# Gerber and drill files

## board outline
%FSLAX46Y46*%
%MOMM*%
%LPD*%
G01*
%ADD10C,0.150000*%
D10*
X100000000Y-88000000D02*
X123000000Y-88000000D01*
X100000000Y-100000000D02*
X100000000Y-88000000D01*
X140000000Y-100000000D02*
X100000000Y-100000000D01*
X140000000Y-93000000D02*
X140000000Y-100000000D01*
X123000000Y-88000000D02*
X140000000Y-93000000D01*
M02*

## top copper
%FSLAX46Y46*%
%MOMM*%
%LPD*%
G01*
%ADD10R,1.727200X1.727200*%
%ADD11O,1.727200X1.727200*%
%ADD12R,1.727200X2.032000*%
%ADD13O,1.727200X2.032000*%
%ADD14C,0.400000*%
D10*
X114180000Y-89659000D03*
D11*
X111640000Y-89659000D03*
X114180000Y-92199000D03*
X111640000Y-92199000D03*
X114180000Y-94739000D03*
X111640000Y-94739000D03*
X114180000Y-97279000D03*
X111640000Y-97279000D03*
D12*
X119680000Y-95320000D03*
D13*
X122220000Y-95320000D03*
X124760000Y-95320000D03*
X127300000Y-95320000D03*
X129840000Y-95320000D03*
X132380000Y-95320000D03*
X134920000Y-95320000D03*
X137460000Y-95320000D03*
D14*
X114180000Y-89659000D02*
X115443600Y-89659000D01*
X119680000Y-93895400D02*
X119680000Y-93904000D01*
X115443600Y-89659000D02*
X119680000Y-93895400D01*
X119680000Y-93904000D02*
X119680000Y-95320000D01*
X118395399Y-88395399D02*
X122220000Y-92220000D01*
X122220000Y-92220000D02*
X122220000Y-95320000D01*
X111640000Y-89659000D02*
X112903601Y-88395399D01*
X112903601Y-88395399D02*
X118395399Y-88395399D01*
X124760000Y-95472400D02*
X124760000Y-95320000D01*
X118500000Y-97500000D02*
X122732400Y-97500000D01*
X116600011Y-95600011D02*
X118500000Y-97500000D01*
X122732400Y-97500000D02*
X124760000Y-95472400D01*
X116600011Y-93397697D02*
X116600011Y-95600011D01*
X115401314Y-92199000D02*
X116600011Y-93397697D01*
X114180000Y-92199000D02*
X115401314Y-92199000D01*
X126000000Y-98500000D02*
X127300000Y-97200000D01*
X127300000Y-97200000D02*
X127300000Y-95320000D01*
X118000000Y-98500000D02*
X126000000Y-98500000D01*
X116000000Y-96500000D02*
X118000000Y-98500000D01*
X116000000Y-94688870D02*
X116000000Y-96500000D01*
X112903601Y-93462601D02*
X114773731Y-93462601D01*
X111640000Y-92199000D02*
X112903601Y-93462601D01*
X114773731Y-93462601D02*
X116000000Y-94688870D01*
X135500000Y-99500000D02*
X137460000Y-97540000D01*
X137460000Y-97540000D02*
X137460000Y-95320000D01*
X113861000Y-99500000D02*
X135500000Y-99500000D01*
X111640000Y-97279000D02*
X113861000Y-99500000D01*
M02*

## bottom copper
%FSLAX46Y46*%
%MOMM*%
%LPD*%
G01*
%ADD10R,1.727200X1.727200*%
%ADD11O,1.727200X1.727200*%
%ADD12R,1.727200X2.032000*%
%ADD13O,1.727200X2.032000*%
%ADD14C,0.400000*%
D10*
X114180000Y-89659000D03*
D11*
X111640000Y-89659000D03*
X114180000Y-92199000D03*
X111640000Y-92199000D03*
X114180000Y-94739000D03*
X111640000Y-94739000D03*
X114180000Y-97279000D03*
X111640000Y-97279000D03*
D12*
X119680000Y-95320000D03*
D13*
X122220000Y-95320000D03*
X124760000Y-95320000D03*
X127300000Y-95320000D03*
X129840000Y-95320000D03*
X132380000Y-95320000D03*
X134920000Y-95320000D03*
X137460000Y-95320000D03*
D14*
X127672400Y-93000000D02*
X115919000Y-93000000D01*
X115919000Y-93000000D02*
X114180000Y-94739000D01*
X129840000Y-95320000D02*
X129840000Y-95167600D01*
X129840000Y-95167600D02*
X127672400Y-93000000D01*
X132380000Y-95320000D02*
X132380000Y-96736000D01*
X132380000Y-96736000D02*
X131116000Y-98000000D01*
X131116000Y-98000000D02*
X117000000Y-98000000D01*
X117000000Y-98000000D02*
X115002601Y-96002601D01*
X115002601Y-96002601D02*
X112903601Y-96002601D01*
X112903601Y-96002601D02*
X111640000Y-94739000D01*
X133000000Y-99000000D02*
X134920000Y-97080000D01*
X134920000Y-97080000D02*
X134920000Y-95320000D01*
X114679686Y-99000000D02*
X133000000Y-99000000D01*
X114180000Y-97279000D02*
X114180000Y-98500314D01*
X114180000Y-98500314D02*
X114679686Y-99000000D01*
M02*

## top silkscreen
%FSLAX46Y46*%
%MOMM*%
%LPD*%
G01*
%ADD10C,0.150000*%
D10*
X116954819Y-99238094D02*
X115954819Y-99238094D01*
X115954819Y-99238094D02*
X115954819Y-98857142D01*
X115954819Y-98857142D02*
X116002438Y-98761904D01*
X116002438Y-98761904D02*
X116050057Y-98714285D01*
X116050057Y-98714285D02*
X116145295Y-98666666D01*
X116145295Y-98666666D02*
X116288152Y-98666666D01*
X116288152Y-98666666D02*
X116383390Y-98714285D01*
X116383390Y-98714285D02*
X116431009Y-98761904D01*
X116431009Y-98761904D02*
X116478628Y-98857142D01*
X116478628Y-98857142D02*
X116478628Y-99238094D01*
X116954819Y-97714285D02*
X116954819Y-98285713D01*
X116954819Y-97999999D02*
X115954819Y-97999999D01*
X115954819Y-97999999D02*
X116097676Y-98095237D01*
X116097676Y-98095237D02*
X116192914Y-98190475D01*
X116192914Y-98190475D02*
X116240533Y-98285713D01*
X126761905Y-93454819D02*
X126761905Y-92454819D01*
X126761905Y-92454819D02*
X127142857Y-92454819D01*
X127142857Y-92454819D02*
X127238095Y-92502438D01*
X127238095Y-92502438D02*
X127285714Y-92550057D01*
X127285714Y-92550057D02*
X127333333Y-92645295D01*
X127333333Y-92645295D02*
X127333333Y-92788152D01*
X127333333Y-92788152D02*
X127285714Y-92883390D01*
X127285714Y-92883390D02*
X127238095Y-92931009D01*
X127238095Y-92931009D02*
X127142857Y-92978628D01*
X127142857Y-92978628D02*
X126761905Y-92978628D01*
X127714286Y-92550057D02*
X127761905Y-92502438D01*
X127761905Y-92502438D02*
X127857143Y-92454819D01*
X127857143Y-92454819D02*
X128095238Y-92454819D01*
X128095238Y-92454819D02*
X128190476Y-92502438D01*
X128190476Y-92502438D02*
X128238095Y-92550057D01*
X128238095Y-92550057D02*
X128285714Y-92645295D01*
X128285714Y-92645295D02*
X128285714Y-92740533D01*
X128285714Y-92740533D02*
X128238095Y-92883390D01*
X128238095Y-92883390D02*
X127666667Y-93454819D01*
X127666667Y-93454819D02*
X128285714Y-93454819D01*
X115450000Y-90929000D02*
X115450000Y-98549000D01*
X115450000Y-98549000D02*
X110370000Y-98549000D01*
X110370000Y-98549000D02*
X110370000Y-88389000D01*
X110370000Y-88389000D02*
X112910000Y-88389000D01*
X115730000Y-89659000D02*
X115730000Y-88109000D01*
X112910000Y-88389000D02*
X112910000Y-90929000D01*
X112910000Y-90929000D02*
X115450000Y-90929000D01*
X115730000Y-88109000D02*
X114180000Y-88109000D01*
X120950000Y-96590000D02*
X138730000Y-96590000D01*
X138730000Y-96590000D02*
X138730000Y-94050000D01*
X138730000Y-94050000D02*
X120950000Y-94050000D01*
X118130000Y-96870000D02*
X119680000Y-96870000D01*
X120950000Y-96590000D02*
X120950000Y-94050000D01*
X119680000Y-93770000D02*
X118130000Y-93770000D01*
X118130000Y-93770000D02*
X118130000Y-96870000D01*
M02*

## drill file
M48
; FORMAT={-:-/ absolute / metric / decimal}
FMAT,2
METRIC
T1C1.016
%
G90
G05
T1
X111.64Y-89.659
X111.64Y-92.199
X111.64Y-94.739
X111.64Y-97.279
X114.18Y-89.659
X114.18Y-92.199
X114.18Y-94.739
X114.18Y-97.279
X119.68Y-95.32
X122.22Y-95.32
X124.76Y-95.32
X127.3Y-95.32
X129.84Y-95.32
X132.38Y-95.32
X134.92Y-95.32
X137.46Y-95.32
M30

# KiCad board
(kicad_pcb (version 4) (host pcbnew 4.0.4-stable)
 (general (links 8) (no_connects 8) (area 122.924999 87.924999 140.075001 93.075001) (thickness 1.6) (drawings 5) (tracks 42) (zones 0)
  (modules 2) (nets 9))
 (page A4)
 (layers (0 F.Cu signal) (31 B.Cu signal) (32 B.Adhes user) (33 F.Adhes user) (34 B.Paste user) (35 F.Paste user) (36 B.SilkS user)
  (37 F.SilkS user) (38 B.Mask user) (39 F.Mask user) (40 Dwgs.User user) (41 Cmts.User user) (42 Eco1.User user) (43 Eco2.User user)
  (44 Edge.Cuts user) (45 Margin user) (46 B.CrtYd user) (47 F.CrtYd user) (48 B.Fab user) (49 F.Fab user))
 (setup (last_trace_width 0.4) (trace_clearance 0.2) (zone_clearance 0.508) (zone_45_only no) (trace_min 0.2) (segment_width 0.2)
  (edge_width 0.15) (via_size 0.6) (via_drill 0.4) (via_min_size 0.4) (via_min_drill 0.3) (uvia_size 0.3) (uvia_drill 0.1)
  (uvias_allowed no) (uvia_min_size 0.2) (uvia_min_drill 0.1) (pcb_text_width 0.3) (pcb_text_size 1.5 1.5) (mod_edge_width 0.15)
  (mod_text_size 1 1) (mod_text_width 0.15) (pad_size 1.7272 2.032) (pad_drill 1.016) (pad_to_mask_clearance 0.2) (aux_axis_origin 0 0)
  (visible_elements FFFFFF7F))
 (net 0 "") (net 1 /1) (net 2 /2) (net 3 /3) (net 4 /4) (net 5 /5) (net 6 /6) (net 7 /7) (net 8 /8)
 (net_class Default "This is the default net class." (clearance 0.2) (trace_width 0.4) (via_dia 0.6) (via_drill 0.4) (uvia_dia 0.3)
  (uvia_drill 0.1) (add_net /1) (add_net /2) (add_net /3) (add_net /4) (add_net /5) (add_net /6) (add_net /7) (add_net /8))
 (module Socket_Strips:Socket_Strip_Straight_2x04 (layer F.Cu) (at 114.18 89.659 270)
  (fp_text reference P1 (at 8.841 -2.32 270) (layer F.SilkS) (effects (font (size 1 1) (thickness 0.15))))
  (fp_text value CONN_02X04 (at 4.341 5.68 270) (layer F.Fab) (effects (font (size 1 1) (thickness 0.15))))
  (fp_line (start 1.27 -1.27) (end 8.89 -1.27) (layer F.SilkS) (width 0.15))
  (fp_line (start 8.89 -1.27) (end 8.89 3.81) (layer F.SilkS) (width 0.15))
  (fp_line (start 8.89 3.81) (end -1.27 3.81) (layer F.SilkS) (width 0.15))
  (fp_line (start -1.27 3.81) (end -1.27 1.27) (layer F.SilkS) (width 0.15))
  (fp_line (start 0 -1.55) (end -1.55 -1.55) (layer F.SilkS) (width 0.15))
  (fp_line (start -1.27 1.27) (end 1.27 1.27) (layer F.SilkS) (width 0.15))
  (fp_line (start 1.27 1.27) (end 1.27 -1.27) (layer F.SilkS) (width 0.15))
  (fp_line (start -1.55 -1.55) (end -1.55 0) (layer F.SilkS) (width 0.15))
  (pad 1 thru_hole rect (at 0 0 270) (size 1.7272 1.7272) (drill 1.016) (layers *.Cu *.Mask) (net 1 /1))
  (pad 2 thru_hole oval (at 0 2.54 270) (size 1.7272 1.7272) (drill 1.016) (layers *.Cu *.Mask) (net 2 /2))
  (pad 3 thru_hole oval (at 2.54 0 270) (size 1.7272 1.7272) (drill 1.016) (layers *.Cu *.Mask) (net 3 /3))
  (pad 4 thru_hole oval (at 2.54 2.54 270) (size 1.7272 1.7272) (drill 1.016) (layers *.Cu *.Mask) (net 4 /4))
  (pad 5 thru_hole oval (at 5.08 0 270) (size 1.7272 1.7272) (drill 1.016) (layers *.Cu *.Mask) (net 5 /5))
  (pad 6 thru_hole oval (at 5.08 2.54 270) (size 1.7272 1.7272) (drill 1.016) (layers *.Cu *.Mask) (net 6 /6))
  (pad 7 thru_hole oval (at 7.62 0 270) (size 1.7272 1.7272) (drill 1.016) (layers *.Cu *.Mask) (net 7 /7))
  (pad 8 thru_hole oval (at 7.62 2.54 270) (size 1.7272 1.7272) (drill 1.016) (layers *.Cu *.Mask) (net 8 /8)))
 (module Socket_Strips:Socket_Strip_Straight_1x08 (layer F.Cu) (at 119.68 95.32)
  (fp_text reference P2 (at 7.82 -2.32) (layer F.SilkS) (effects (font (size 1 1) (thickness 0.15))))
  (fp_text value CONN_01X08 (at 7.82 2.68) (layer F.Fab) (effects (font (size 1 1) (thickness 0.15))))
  (fp_line (start 1.27 1.27) (end 19.05 1.27) (layer F.SilkS) (width 0.15))
  (fp_line (start 19.05 1.27) (end 19.05 -1.27) (layer F.SilkS) (width 0.15))
  (fp_line (start 19.05 -1.27) (end 1.27 -1.27) (layer F.SilkS) (width 0.15))
  (fp_line (start -1.55 1.55) (end 0 1.55) (layer F.SilkS) (width 0.15))
  (fp_line (start 1.27 1.27) (end 1.27 -1.27) (layer F.SilkS) (width 0.15))
  (fp_line (start 0 -1.55) (end -1.55 -1.55) (layer F.SilkS) (width 0.15))
  (fp_line (start -1.55 -1.55) (end -1.55 1.55) (layer F.SilkS) (width 0.15))
  (pad 1 thru_hole rect (at 0 0) (size 1.7272 2.032) (drill 1.016) (layers *.Cu *.Mask) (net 1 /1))
  (pad 2 thru_hole oval (at 2.54 0) (size 1.7272 2.032) (drill 1.016) (layers *.Cu *.Mask) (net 2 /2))
  (pad 3 thru_hole oval (at 5.08 0) (size 1.7272 2.032) (drill 1.016) (layers *.Cu *.Mask) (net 3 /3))
  (pad 4 thru_hole oval (at 7.62 0) (size 1.7272 2.032) (drill 1.016) (layers *.Cu *.Mask) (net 4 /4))
  (pad 5 thru_hole oval (at 10.16 0) (size 1.7272 2.032) (drill 1.016) (layers *.Cu *.Mask) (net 5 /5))
  (pad 6 thru_hole oval (at 12.7 0) (size 1.7272 2.032) (drill 1.016) (layers *.Cu *.Mask) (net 6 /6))
  (pad 7 thru_hole oval (at 15.24 0) (size 1.7272 2.032) (drill 1.016) (layers *.Cu *.Mask) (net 7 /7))
  (pad 8 thru_hole oval (at 17.78 0) (size 1.7272 2.032) (drill 1.016) (layers *.Cu *.Mask) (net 8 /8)))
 (gr_line (start 100 88) (end 123 88) (layer Edge.Cuts) (width 0.15))
 (gr_line (start 100 100) (end 100 88) (layer Edge.Cuts) (width 0.15))
 (gr_line (start 140 100) (end 100 100) (layer Edge.Cuts) (width 0.15))
 (gr_line (start 140 93) (end 140 100) (layer Edge.Cuts) (width 0.15))
 (gr_line (start 123 88) (end 140 93) (layer Edge.Cuts) (width 0.15))
 (segment (start 114.18 89.659) (end 115.4436 89.659) (width 0.4) (layer F.Cu) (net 1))
 (segment (start 119.68 93.8954) (end 119.68 93.904) (width 0.4) (layer F.Cu) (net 1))
 (segment (start 115.4436 89.659) (end 119.68 93.8954) (width 0.4) (layer F.Cu) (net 1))
 (segment (start 119.68 93.904) (end 119.68 95.32) (width 0.4) (layer F.Cu) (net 1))
 (segment (start 118.395399 88.395399) (end 122.22 92.22) (width 0.4) (layer F.Cu) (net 2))
 (segment (start 122.22 92.22) (end 122.22 95.32) (width 0.4) (layer F.Cu) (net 2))
 (segment (start 111.64 89.659) (end 112.903601 88.395399) (width 0.4) (layer F.Cu) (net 2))
 (segment (start 112.903601 88.395399) (end 118.395399 88.395399) (width 0.4) (layer F.Cu) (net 2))
 (segment (start 124.76 95.4724) (end 124.76 95.32) (width 0.4) (layer F.Cu) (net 3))
 (segment (start 118.5 97.5) (end 122.7324 97.5) (width 0.4) (layer F.Cu) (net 3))
 (segment (start 116.600011 95.600011) (end 118.5 97.5) (width 0.4) (layer F.Cu) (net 3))
 (segment (start 122.7324 97.5) (end 124.76 95.4724) (width 0.4) (layer F.Cu) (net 3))
 (segment (start 116.600011 93.397697) (end 116.600011 95.600011) (width 0.4) (layer F.Cu) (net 3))
 (segment (start 115.401314 92.199) (end 116.600011 93.397697) (width 0.4) (layer F.Cu) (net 3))
 (segment (start 114.18 92.199) (end 115.401314 92.199) (width 0.4) (layer F.Cu) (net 3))
 (segment (start 126 98.5) (end 127.3 97.2) (width 0.4) (layer F.Cu) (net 4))
 (segment (start 127.3 97.2) (end 127.3 95.32) (width 0.4) (layer F.Cu) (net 4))
 (segment (start 118 98.5) (end 126 98.5) (width 0.4) (layer F.Cu) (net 4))
 (segment (start 116 96.5) (end 118 98.5) (width 0.4) (layer F.Cu) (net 4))
 (segment (start 116 94.68887) (end 116 96.5) (width 0.4) (layer F.Cu) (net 4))
 (segment (start 112.903601 93.462601) (end 114.773731 93.462601) (width 0.4) (layer F.Cu) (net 4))
 (segment (start 111.64 92.199) (end 112.903601 93.462601) (width 0.4) (layer F.Cu) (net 4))
 (segment (start 114.773731 93.462601) (end 116 94.68887) (width 0.4) (layer F.Cu) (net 4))
 (segment (start 127.6724 93) (end 115.919 93) (width 0.4) (layer B.Cu) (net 5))
 (segment (start 115.919 93) (end 114.18 94.739) (width 0.4) (layer B.Cu) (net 5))
 (segment (start 129.84 95.32) (end 129.84 95.1676) (width 0.4) (layer B.Cu) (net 5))
 (segment (start 129.84 95.1676) (end 127.6724 93) (width 0.4) (layer B.Cu) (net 5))
 (segment (start 132.38 95.32) (end 132.38 96.736) (width 0.4) (layer B.Cu) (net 6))
 (segment (start 132.38 96.736) (end 131.116 98) (width 0.4) (layer B.Cu) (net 6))
 (segment (start 131.116 98) (end 117 98) (width 0.4) (layer B.Cu) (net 6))
 (segment (start 117 98) (end 115.002601 96.002601) (width 0.4) (layer B.Cu) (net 6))
 (segment (start 115.002601 96.002601) (end 112.903601 96.002601) (width 0.4) (layer B.Cu) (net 6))
 (segment (start 112.903601 96.002601) (end 111.64 94.739) (width 0.4) (layer B.Cu) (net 6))
 (segment (start 133 99) (end 134.92 97.08) (width 0.4) (layer B.Cu) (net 7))
 (segment (start 134.92 97.08) (end 134.92 95.32) (width 0.4) (layer B.Cu) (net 7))
 (segment (start 114.679686 99) (end 133 99) (width 0.4) (layer B.Cu) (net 7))
 (segment (start 114.18 97.279) (end 114.18 98.500314) (width 0.4) (layer B.Cu) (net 7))
 (segment (start 114.18 98.500314) (end 114.679686 99) (width 0.4) (layer B.Cu) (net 7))
 (segment (start 135.5 99.5) (end 137.46 97.54) (width 0.4) (layer F.Cu) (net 8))
 (segment (start 137.46 97.54) (end 137.46 95.32) (width 0.4) (layer F.Cu) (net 8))
 (segment (start 113.861 99.5) (end 135.5 99.5) (width 0.4) (layer F.Cu) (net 8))
 (segment (start 111.64 97.279) (end 113.861 99.5) (width 0.4) (layer F.Cu) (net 8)))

